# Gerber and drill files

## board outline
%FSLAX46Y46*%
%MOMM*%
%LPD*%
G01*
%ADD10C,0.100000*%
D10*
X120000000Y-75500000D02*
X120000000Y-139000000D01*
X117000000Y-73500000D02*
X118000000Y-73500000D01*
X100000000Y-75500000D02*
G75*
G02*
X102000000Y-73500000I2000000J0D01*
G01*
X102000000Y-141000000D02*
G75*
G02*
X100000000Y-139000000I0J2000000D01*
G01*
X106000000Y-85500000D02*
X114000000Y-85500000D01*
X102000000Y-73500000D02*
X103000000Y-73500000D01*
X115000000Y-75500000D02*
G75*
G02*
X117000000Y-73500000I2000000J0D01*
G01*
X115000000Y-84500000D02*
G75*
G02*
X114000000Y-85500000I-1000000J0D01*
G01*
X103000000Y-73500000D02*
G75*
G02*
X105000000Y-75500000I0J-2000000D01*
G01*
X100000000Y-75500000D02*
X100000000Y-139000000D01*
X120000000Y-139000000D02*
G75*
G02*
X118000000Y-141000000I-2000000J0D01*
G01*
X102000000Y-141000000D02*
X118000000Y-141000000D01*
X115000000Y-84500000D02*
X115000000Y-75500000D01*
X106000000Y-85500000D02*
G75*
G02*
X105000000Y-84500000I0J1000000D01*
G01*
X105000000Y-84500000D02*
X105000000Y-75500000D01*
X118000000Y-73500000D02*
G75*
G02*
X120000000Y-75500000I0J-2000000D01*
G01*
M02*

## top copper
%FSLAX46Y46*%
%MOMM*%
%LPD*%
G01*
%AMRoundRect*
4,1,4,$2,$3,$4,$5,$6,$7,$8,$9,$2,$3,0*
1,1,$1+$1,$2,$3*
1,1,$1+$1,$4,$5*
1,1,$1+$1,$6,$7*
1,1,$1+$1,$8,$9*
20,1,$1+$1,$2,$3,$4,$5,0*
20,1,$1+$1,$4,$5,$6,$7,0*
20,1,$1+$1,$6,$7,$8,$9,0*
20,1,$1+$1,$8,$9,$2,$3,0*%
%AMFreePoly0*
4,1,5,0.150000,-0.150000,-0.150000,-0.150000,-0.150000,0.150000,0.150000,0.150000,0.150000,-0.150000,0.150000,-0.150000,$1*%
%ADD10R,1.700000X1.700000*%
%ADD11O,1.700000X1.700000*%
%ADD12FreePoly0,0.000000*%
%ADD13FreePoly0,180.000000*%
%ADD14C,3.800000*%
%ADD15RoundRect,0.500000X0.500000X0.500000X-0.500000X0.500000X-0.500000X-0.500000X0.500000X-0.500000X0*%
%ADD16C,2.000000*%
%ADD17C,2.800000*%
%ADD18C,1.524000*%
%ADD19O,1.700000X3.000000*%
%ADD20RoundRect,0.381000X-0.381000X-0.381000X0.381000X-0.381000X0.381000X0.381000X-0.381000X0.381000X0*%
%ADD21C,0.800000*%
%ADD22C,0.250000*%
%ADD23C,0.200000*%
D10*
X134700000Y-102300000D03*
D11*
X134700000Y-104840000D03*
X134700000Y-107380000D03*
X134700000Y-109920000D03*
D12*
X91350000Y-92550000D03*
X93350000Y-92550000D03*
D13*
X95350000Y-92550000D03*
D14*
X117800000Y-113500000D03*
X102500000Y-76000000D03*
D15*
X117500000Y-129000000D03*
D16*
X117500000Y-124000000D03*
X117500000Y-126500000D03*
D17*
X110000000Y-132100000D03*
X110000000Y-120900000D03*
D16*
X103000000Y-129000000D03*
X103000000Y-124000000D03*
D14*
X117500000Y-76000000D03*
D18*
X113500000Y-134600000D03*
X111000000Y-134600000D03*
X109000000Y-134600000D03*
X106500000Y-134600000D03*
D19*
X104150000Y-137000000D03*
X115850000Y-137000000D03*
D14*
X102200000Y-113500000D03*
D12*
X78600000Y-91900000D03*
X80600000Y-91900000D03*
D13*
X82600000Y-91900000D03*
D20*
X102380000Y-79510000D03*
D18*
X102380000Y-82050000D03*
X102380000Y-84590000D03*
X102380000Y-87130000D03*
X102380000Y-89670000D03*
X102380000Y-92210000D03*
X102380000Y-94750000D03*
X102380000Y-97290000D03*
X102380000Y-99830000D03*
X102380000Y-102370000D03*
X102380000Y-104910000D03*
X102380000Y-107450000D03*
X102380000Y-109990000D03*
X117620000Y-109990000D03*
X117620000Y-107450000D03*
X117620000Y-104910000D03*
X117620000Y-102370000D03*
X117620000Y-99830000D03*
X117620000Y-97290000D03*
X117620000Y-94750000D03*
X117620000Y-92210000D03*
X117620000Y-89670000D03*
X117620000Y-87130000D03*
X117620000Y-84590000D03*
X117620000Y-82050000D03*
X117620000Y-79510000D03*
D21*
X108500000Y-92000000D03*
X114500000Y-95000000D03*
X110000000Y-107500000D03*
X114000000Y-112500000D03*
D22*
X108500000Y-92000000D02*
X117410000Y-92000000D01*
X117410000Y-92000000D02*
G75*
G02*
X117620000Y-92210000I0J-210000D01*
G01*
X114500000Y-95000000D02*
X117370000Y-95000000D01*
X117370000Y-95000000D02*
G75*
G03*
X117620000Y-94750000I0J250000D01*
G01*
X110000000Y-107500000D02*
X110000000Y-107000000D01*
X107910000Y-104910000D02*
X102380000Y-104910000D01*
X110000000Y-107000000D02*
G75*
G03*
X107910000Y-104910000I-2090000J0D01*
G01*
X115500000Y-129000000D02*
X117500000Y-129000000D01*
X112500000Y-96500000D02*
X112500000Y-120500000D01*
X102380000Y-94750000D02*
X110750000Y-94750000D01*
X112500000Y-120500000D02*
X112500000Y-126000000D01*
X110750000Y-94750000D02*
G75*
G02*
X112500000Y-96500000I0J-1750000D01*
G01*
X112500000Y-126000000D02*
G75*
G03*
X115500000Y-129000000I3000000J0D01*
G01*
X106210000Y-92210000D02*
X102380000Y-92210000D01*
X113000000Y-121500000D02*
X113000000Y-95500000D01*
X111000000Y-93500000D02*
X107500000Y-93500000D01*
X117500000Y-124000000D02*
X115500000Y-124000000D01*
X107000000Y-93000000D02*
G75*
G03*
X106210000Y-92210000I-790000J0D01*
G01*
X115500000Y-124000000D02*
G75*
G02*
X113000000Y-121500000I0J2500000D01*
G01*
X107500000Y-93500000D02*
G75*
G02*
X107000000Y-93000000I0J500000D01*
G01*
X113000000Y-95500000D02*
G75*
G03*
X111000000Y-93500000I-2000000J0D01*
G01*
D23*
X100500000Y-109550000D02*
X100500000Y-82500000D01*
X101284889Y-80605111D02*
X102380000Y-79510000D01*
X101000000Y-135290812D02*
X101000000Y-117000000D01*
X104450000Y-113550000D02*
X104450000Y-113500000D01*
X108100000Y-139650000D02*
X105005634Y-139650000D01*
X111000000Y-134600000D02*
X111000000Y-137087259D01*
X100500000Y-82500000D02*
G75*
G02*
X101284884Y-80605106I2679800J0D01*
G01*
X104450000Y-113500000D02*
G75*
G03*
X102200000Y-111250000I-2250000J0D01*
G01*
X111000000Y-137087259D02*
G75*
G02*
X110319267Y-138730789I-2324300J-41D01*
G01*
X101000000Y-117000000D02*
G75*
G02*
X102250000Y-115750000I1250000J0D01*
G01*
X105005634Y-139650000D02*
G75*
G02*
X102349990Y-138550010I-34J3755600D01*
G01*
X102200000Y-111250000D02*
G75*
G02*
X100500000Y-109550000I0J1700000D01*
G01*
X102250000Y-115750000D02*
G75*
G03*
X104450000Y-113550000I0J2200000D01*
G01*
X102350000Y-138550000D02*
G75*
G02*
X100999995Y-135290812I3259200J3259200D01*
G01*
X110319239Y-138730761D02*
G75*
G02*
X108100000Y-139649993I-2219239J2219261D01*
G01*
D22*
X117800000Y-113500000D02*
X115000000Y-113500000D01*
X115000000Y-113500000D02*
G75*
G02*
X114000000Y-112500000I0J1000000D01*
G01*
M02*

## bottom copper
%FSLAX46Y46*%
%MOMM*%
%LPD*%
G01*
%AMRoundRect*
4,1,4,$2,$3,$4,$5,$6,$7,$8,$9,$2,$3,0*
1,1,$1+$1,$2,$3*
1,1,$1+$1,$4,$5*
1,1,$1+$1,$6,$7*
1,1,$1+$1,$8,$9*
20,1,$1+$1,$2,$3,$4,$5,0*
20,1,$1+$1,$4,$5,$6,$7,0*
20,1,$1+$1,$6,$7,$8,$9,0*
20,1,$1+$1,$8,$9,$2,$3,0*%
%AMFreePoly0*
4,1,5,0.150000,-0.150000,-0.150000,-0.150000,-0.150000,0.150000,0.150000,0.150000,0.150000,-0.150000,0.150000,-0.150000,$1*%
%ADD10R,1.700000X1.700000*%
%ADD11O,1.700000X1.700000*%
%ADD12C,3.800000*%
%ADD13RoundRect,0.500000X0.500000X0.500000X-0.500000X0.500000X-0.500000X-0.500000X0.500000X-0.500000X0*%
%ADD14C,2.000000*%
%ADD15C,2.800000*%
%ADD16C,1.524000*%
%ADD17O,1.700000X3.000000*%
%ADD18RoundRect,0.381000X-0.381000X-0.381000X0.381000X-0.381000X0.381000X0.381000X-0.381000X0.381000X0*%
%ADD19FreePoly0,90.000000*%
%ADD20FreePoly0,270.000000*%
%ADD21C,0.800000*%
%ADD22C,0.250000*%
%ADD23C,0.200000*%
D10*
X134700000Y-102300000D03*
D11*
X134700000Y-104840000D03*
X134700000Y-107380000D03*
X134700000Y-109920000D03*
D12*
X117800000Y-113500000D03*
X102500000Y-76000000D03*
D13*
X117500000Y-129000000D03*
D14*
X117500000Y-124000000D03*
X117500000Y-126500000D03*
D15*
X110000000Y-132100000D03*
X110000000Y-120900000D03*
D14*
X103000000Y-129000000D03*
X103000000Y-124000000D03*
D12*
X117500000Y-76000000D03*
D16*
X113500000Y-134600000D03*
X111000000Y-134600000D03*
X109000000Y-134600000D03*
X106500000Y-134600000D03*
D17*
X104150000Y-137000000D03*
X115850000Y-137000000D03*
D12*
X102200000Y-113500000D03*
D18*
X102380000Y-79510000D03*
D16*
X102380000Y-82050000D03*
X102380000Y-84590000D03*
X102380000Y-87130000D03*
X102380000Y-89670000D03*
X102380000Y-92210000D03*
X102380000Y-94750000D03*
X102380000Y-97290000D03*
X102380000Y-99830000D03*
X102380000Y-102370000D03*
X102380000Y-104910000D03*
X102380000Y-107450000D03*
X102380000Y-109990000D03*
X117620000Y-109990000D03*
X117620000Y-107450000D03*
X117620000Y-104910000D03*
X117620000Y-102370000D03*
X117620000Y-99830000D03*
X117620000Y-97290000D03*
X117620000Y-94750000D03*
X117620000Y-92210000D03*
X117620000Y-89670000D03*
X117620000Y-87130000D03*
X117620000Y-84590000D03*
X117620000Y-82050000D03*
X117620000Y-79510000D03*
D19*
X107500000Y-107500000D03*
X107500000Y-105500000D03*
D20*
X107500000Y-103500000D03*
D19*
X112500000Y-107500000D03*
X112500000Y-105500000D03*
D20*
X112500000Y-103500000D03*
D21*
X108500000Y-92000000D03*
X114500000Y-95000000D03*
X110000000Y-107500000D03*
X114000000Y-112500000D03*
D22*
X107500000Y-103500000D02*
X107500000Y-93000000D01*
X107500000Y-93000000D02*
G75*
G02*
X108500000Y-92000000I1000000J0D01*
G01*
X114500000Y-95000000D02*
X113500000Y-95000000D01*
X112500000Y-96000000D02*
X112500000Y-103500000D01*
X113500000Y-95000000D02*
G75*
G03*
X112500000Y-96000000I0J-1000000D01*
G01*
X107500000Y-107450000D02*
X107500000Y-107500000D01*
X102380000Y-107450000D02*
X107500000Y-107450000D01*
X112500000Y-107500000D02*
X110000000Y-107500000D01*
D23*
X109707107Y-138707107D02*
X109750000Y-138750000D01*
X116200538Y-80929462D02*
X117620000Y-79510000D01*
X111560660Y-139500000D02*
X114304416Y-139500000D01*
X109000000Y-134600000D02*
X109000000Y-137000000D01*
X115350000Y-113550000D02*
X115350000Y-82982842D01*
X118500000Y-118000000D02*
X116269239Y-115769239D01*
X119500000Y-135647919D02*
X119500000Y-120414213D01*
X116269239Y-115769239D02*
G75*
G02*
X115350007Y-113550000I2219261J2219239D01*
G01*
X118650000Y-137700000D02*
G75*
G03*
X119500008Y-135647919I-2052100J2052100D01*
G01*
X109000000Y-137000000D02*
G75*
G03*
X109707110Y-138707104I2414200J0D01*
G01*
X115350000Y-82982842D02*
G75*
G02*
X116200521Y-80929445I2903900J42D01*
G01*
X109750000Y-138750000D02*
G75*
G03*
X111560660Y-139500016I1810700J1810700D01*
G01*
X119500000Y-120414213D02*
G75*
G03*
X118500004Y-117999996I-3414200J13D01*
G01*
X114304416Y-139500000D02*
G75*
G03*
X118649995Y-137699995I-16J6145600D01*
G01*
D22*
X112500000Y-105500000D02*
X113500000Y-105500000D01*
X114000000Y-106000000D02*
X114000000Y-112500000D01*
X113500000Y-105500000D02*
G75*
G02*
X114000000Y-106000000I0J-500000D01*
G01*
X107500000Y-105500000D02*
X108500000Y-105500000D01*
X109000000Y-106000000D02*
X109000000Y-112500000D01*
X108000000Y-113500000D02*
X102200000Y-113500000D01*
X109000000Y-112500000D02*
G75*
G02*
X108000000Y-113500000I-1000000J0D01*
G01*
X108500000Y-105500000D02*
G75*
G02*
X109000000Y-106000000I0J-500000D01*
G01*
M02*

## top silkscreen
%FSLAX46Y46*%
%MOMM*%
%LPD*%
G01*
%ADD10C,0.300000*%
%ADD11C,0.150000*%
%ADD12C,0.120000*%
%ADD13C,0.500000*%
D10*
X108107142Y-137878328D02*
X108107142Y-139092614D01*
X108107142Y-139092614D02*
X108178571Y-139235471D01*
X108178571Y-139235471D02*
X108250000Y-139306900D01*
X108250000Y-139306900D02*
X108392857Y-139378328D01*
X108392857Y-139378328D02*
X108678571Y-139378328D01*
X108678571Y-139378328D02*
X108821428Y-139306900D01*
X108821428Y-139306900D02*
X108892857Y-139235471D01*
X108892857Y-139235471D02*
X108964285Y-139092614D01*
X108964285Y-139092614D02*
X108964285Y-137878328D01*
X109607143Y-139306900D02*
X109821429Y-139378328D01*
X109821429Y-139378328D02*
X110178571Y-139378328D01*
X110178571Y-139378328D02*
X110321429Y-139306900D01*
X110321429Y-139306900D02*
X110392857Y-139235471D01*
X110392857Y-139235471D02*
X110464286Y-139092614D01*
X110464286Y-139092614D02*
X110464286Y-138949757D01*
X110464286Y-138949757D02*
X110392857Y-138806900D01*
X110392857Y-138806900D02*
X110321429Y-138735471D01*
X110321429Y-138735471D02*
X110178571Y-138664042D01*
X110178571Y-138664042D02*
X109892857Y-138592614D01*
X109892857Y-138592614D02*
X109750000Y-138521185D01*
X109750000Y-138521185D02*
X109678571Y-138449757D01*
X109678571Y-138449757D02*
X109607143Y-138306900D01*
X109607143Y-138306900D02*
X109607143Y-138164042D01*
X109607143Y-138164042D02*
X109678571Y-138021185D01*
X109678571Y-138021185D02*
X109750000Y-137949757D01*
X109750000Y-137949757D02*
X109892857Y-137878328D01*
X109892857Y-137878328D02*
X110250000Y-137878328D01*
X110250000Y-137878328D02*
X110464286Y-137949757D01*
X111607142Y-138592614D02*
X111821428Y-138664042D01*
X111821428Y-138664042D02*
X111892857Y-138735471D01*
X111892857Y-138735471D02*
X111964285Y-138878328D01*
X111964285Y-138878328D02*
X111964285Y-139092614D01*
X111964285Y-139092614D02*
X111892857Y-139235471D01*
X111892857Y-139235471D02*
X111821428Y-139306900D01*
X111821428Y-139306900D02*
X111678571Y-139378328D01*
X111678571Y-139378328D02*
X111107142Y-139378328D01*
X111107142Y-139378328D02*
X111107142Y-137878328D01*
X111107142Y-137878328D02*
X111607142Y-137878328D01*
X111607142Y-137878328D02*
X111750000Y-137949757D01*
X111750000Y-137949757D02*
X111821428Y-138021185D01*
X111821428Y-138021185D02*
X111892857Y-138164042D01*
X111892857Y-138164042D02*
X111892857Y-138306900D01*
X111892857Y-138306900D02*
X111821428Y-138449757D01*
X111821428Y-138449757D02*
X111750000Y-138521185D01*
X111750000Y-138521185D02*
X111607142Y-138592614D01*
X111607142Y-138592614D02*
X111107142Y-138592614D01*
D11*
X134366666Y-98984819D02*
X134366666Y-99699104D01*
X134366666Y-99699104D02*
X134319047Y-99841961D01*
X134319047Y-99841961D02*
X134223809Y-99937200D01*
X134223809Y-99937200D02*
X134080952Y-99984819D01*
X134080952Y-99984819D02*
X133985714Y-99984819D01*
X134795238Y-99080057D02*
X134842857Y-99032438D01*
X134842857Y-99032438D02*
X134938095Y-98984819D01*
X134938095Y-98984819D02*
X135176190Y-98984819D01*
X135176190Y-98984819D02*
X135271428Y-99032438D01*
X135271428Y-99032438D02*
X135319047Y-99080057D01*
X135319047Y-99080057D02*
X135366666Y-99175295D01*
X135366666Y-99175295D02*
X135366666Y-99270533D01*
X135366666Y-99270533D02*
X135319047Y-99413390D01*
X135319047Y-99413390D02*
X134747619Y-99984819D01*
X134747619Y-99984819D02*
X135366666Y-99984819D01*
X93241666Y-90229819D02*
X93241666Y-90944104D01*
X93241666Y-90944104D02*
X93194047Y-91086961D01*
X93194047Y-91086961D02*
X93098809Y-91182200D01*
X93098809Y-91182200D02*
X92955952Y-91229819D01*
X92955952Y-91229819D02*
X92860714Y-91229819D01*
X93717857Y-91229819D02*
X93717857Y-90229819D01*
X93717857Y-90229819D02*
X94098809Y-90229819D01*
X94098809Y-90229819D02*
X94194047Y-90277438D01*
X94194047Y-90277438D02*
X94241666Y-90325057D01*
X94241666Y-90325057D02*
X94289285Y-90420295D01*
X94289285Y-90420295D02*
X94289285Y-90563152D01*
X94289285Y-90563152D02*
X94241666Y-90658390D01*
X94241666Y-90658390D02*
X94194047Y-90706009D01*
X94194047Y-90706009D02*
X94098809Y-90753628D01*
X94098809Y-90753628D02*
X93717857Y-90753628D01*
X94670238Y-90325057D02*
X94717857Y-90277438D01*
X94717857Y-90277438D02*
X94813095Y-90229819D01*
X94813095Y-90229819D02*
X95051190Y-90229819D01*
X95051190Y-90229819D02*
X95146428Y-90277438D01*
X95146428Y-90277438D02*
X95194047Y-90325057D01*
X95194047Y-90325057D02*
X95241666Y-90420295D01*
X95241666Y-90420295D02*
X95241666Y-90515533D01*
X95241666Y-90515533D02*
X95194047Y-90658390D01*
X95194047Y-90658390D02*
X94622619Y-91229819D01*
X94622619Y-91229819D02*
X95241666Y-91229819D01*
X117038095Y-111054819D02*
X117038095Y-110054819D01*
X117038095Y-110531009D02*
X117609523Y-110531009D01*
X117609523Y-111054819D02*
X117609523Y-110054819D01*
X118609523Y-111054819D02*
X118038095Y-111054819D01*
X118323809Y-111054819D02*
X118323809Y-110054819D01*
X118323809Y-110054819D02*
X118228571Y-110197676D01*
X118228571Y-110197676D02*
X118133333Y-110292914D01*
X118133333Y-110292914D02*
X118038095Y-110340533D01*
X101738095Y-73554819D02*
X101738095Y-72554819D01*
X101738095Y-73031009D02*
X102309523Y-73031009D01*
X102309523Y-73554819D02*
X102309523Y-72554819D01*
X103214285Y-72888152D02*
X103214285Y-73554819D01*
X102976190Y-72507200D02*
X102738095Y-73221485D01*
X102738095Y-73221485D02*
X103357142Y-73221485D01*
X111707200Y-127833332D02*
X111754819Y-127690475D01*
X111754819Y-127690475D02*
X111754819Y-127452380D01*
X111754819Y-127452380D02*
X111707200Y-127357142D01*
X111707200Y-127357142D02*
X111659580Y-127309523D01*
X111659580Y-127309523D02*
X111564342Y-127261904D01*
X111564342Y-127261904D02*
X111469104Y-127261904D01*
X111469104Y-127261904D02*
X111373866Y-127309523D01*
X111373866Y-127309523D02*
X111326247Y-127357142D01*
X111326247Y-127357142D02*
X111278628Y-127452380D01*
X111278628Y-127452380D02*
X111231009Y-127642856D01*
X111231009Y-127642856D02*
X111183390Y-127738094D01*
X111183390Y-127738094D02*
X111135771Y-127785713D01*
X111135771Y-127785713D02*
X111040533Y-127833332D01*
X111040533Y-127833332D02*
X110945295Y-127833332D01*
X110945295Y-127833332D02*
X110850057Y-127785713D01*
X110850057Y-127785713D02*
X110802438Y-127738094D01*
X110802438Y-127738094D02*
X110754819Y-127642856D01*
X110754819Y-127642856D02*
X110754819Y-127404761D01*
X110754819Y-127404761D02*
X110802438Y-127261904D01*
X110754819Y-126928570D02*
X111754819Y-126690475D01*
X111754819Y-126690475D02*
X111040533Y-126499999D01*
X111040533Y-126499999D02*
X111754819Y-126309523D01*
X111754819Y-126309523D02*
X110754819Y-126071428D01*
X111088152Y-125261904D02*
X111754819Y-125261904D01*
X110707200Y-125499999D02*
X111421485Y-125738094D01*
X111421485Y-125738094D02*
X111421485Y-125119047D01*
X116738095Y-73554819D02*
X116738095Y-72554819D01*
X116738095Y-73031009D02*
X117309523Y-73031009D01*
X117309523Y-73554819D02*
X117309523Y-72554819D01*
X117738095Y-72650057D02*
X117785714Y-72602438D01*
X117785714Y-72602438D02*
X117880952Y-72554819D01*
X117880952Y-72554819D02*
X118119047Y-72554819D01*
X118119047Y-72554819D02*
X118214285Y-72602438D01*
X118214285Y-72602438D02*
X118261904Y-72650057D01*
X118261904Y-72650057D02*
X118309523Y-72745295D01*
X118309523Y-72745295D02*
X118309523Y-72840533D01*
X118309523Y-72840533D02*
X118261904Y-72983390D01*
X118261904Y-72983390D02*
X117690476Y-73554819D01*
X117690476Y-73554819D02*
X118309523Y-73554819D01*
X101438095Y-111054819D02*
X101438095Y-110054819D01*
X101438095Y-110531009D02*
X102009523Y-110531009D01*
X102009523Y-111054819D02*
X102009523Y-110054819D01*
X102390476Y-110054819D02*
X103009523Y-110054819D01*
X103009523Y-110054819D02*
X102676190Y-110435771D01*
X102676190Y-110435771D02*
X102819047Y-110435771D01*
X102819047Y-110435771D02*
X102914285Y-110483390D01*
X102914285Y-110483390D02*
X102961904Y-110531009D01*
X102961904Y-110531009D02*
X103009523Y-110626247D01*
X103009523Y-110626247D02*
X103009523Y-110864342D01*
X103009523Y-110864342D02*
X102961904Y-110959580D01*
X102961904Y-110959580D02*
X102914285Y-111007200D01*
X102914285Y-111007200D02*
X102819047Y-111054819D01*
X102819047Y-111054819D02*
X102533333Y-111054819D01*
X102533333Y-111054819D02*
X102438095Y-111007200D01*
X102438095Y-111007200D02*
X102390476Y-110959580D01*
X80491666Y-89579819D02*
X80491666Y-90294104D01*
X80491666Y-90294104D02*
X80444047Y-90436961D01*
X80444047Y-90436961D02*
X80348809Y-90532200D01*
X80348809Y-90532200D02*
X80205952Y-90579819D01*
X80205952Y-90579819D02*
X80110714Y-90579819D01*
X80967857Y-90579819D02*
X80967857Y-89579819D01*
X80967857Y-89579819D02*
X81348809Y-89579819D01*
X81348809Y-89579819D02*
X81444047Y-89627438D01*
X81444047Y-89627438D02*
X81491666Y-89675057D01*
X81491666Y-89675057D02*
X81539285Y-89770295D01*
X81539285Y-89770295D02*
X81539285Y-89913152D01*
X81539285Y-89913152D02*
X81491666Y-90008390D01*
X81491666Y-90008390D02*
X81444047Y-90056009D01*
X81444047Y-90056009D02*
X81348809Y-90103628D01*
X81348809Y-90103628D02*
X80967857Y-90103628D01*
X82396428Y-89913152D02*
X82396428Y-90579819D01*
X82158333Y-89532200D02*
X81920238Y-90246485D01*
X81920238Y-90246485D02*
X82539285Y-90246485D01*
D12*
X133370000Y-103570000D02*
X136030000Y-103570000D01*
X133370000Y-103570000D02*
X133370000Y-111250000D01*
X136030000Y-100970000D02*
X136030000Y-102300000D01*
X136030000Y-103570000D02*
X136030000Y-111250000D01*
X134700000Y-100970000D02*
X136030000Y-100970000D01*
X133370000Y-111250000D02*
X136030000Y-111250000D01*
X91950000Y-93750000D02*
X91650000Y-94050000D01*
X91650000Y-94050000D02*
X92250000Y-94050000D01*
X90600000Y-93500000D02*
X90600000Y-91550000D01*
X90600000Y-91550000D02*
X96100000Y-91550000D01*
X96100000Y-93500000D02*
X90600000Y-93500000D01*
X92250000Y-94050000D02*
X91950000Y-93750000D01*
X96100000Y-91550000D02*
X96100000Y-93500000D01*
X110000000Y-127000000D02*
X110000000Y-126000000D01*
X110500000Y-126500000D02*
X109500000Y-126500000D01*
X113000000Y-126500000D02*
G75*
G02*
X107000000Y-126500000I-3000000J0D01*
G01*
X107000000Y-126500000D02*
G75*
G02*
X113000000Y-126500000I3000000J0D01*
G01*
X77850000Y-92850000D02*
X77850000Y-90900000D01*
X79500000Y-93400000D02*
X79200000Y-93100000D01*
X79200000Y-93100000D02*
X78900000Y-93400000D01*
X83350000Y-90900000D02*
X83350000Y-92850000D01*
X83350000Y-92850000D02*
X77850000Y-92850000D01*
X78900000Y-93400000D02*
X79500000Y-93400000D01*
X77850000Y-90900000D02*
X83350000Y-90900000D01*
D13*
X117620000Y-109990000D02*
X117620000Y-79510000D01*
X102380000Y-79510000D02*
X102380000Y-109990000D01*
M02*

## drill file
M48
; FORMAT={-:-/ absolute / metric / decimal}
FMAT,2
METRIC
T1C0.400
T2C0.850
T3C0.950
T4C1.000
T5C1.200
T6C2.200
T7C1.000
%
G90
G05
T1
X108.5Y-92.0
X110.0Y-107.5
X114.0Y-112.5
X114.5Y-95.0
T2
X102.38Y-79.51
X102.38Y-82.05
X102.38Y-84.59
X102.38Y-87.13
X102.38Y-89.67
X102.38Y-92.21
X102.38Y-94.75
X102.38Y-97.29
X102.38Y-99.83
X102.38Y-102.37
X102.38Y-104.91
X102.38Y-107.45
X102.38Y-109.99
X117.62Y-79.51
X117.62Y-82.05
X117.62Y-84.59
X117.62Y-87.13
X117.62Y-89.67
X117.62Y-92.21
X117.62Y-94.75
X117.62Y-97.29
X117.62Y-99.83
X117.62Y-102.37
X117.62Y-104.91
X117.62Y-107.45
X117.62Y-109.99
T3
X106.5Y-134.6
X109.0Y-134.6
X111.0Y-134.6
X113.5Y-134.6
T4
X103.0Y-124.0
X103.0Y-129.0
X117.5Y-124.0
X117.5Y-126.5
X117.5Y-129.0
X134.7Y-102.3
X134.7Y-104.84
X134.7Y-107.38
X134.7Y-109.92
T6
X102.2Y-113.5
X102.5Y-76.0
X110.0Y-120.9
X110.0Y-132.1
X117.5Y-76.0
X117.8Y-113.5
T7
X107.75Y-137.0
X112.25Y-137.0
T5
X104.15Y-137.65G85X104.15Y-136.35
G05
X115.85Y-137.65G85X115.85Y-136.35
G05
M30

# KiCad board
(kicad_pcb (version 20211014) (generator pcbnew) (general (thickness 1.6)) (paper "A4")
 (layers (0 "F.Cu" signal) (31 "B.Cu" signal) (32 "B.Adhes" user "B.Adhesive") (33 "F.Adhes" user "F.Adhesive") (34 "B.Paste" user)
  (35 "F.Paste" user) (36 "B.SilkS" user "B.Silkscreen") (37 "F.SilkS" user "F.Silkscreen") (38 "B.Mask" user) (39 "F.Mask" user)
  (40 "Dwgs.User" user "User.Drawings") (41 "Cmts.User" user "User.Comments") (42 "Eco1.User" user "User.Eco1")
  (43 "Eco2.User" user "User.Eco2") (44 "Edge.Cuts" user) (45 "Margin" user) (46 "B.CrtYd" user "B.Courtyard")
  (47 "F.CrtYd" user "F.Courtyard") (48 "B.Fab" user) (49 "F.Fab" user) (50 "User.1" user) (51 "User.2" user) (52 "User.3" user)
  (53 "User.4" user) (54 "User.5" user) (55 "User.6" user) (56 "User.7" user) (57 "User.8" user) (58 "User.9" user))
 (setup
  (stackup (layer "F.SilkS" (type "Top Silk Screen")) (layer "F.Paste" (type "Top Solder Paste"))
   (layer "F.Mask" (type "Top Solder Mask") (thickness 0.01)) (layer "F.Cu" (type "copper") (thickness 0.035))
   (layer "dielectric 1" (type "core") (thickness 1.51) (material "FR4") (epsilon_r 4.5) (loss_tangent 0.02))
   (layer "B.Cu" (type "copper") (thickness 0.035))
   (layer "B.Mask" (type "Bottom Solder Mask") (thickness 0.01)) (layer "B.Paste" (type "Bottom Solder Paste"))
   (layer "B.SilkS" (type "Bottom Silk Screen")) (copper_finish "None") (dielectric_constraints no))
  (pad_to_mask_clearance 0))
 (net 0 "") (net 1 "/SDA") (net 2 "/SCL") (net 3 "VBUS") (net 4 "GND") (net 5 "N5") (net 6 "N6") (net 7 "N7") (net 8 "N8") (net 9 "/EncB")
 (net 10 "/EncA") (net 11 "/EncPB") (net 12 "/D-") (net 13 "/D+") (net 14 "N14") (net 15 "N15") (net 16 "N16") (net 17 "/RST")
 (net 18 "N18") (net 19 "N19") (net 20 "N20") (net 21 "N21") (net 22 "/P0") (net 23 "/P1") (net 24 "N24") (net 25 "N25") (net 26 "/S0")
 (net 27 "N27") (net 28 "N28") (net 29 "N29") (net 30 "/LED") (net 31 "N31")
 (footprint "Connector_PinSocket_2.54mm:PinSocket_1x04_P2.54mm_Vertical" (layer "F.Cu") (at 134.7 102.3)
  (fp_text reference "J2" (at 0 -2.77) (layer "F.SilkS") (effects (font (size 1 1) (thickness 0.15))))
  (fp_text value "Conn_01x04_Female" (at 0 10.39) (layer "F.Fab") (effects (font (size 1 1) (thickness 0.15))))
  (fp_line (start -1.33 1.27) (end 1.33 1.27) (layer "F.SilkS") (width 0.12))
  (fp_line (start -1.33 1.27) (end -1.33 8.95) (layer "F.SilkS") (width 0.12))
  (fp_line (start 1.33 -1.33) (end 1.33 0) (layer "F.SilkS") (width 0.12))
  (fp_line (start 1.33 1.27) (end 1.33 8.95) (layer "F.SilkS") (width 0.12))
  (fp_line (start 0 -1.33) (end 1.33 -1.33) (layer "F.SilkS") (width 0.12))
  (fp_line (start -1.33 8.95) (end 1.33 8.95) (layer "F.SilkS") (width 0.12))
  (pad "1" thru_hole rect (at 0 0) (size 1.7 1.7) (drill 1) (layers *.Cu *.Mask) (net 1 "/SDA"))
  (pad "2" thru_hole oval (at 0 2.54) (size 1.7 1.7) (drill 1) (layers *.Cu *.Mask) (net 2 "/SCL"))
  (pad "3" thru_hole oval (at 0 5.08) (size 1.7 1.7) (drill 1) (layers *.Cu *.Mask) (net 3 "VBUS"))
  (pad "4" thru_hole oval (at 0 7.62) (size 1.7 1.7) (drill 1) (layers *.Cu *.Mask) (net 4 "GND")))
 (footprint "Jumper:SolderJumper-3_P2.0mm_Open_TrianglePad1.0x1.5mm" (layer "F.Cu") (at 93.35 92.55)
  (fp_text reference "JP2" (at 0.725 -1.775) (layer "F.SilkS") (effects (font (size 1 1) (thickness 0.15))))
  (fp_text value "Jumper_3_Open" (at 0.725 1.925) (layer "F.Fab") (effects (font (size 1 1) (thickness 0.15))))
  (fp_line (start -1.4 1.2) (end -1.7 1.5) (layer "F.SilkS") (width 0.12))
  (fp_line (start -1.7 1.5) (end -1.1 1.5) (layer "F.SilkS") (width 0.12))
  (fp_line (start -2.75 0.95) (end -2.75 -1) (layer "F.SilkS") (width 0.12))
  (fp_line (start -2.75 -1) (end 2.75 -1) (layer "F.SilkS") (width 0.12))
  (fp_line (start 2.75 0.95) (end -2.75 0.95) (layer "F.SilkS") (width 0.12))
  (fp_line (start -1.1 1.5) (end -1.4 1.2) (layer "F.SilkS") (width 0.12))
  (fp_line (start 2.75 -1) (end 2.75 0.95) (layer "F.SilkS") (width 0.12))
  (pad "" smd rect (at 1.2 0) (size 1.5 1.5) (layers "F.Mask"))
  (pad "" smd rect (at -1.2 0) (size 1.5 1.5) (layers "F.Mask"))
  (pad "1" smd custom (at -2 0) (size 0.3 0.3) (layers "F.Cu" "F.Mask") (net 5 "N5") (zone_connect 2)
   (options (clearance outline) (anchor rect)) (primitives))
  (pad "2" smd custom (at 0 0) (size 0.3 0.3) (layers "F.Cu") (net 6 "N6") (zone_connect 2) (options (clearance outline) (anchor rect))
   (primitives))
  (pad "3" smd custom (at 2 0 180) (size 0.3 0.3) (layers "F.Cu" "F.Mask") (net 3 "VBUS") (zone_connect 2)
   (options (clearance outline) (anchor rect)) (primitives)))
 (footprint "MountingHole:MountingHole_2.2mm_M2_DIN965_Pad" (layer "F.Cu") (at 117.8 113.5)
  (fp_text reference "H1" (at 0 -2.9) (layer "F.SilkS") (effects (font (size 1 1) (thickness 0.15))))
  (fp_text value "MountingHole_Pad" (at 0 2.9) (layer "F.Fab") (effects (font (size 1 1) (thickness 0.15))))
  (pad "1" thru_hole circle (at 0 0) (size 3.8 3.8) (drill 2.2) (layers *.Cu *.Mask) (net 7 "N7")))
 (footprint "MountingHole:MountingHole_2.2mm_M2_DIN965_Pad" (layer "F.Cu") (at 102.5 76)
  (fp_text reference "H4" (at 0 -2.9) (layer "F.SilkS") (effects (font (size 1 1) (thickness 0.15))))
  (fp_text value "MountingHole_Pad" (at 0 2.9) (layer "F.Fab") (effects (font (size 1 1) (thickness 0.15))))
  (pad "1" thru_hole circle (at 0 0) (size 3.8 3.8) (drill 2.2) (layers *.Cu *.Mask) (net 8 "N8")))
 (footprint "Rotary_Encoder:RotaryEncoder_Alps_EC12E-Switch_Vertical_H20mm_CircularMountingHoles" (layer "F.Cu") (at 117.5 129 180)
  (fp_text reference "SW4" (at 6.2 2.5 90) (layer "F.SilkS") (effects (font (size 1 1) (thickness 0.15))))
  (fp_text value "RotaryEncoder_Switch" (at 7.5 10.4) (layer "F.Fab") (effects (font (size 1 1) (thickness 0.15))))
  (fp_line (start 7.5 2) (end 7.5 3) (layer "F.SilkS") (width 0.12))
  (fp_line (start 7 2.5) (end 8 2.5) (layer "F.SilkS") (width 0.12))
  (fp_circle (center 7.5 2.5) (end 10.5 2.5) (layer "F.SilkS") (width 0.12) (fill none))
  (pad "A" thru_hole roundrect (at 0 0 180) (size 2 2) (drill 1) (layers *.Cu *.Mask) (roundrect_rratio 0.25) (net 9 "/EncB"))
  (pad "B" thru_hole circle (at 0 5 180) (size 2 2) (drill 1) (layers *.Cu *.Mask) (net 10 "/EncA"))
  (pad "C" thru_hole circle (at 0 2.5 180) (size 2 2) (drill 1) (layers *.Cu *.Mask) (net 4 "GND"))
  (pad "MP" thru_hole circle (at 7.5 -3.1 180) (size 2.8 2.8) (drill 2.2) (layers *.Cu *.Mask))
  (pad "MP" thru_hole circle (at 7.5 8.1 180) (size 2.8 2.8) (drill 2.2) (layers *.Cu *.Mask))
  (pad "S1" thru_hole circle (at 14.5 0 180) (size 2 2) (drill 1) (layers *.Cu *.Mask) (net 4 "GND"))
  (pad "S2" thru_hole circle (at 14.5 5 180) (size 2 2) (drill 1) (layers *.Cu *.Mask) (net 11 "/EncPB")))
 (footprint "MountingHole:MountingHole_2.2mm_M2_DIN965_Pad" (layer "F.Cu") (at 117.5 76)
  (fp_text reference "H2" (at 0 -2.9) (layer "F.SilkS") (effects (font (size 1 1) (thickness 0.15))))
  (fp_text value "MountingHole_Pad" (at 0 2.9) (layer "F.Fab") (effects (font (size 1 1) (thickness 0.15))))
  (pad "1" thru_hole circle (at 0 0) (size 3.8 3.8) (drill 2.2) (layers *.Cu *.Mask) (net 6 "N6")))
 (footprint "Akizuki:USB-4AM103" (layer "F.Cu") (at 110 136 180)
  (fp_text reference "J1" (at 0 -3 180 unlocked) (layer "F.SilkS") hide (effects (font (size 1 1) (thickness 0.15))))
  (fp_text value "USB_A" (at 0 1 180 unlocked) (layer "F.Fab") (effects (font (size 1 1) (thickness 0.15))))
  (pad "" np_thru_hole circle (at 2.25 -1 180) (size 1 1) (drill 1) (layers *.Mask))
  (pad "" np_thru_hole circle (at -2.25 -1 180) (size 1 1) (drill 1) (layers *.Mask))
  (pad "1" thru_hole circle (at -3.5 1.4 180) (size 1.524 1.524) (drill 0.95) (layers *.Cu *.Mask) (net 3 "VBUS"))
  (pad "2" thru_hole circle (at -1 1.4 180) (size 1.524 1.524) (drill 0.95) (layers *.Cu *.Mask) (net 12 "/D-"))
  (pad "3" thru_hole circle (at 1 1.4 180) (size 1.524 1.524) (drill 0.95) (layers *.Cu *.Mask) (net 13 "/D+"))
  (pad "4" thru_hole circle (at 3.5 1.4 180) (size 1.524 1.524) (drill 0.95) (layers *.Cu *.Mask) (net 4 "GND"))
  (pad "5" thru_hole oval (at 5.85 -1 180) (size 1.7 3) (drill oval 1.2 2.5) (layers *.Cu *.Mask) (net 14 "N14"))
  (pad "5" thru_hole oval (at -5.85 -1 180) (size 1.7 3) (drill oval 1.2 2.5) (layers *.Cu *.Mask) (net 14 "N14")))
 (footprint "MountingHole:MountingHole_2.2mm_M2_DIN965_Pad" (layer "F.Cu") (at 102.2 113.5)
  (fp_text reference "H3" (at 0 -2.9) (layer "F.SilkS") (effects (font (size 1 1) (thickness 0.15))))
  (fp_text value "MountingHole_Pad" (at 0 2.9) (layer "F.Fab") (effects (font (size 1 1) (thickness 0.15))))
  (pad "1" thru_hole circle (at 0 0) (size 3.8 3.8) (drill 2.2) (layers *.Cu *.Mask) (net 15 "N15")))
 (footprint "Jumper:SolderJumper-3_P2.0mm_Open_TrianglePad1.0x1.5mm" (layer "F.Cu") (at 80.6 91.9)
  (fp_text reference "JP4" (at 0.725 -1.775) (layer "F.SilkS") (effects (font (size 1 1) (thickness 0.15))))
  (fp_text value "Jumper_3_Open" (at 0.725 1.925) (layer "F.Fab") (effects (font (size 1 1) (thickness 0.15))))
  (fp_line (start -2.75 0.95) (end -2.75 -1) (layer "F.SilkS") (width 0.12))
  (fp_line (start -1.1 1.5) (end -1.4 1.2) (layer "F.SilkS") (width 0.12))
  (fp_line (start -1.4 1.2) (end -1.7 1.5) (layer "F.SilkS") (width 0.12))
  (fp_line (start 2.75 -1) (end 2.75 0.95) (layer "F.SilkS") (width 0.12))
  (fp_line (start 2.75 0.95) (end -2.75 0.95) (layer "F.SilkS") (width 0.12))
  (fp_line (start -1.7 1.5) (end -1.1 1.5) (layer "F.SilkS") (width 0.12))
  (fp_line (start -2.75 -1) (end 2.75 -1) (layer "F.SilkS") (width 0.12))
  (pad "" smd rect (at -1.2 0) (size 1.5 1.5) (layers "F.Mask"))
  (pad "" smd rect (at 1.2 0) (size 1.5 1.5) (layers "F.Mask"))
  (pad "1" smd custom (at -2 0) (size 0.3 0.3) (layers "F.Cu" "F.Mask") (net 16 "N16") (zone_connect 2)
   (options (clearance outline) (anchor rect)) (primitives))
  (pad "2" smd custom (at 0 0) (size 0.3 0.3) (layers "F.Cu") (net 8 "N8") (zone_connect 2) (options (clearance outline) (anchor rect))
   (primitives))
  (pad "3" smd custom (at 2 0 180) (size 0.3 0.3) (layers "F.Cu" "F.Mask") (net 4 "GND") (zone_connect 2)
   (options (clearance outline) (anchor rect)) (primitives)))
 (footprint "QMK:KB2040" (layer "F.Cu") (at 110 94.75)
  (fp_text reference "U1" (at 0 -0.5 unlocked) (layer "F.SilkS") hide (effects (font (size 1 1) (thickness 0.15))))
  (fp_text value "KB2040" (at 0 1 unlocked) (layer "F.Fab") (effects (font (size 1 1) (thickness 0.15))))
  (fp_line (start 7.62 15.24) (end 7.62 -15.24) (layer "F.SilkS") (width 0.5))
  (fp_line (start -7.62 -15.24) (end -7.62 15.24) (layer "F.SilkS") (width 0.5))
  (pad "0" thru_hole roundrect (at -7.62 -15.24) (size 1.524 1.524) (drill 0.85) (layers *.Cu *.Mask) (roundrect_rratio 0.25) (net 12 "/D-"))
  (pad "1" thru_hole circle (at -7.62 -12.7) (size 1.524 1.524) (drill 0.85) (layers *.Cu *.Mask) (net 3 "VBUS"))
  (pad "2" thru_hole circle (at -7.62 -10.16) (size 1.524 1.524) (drill 0.85) (layers *.Cu *.Mask) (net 4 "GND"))
  (pad "3" thru_hole circle (at -7.62 -7.62) (size 1.524 1.524) (drill 0.85) (layers *.Cu *.Mask) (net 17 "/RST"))
  (pad "4" thru_hole circle (at -7.62 -5.08) (size 1.524 1.524) (drill 0.85) (layers *.Cu *.Mask) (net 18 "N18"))
  (pad "5" thru_hole circle (at -7.62 -2.54) (size 1.524 1.524) (drill 0.85) (layers *.Cu *.Mask) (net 10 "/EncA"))
  (pad "6" thru_hole circle (at -7.62 0) (size 1.524 1.524) (drill 0.85) (layers *.Cu *.Mask) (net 9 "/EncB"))
  (pad "7" thru_hole circle (at -7.62 2.54) (size 1.524 1.524) (drill 0.85) (layers *.Cu *.Mask) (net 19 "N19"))
  (pad "8" thru_hole circle (at -7.62 5.08) (size 1.524 1.524) (drill 0.85) (layers *.Cu *.Mask) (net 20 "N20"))
  (pad "9" thru_hole circle (at -7.62 7.62) (size 1.524 1.524) (drill 0.85) (layers *.Cu *.Mask) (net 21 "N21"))
  (pad "10" thru_hole circle (at -7.62 10.16) (size 1.524 1.524) (drill 0.85) (layers *.Cu *.Mask) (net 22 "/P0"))
  (pad "11" thru_hole circle (at -7.62 12.7) (size 1.524 1.524) (drill 0.85) (layers *.Cu *.Mask) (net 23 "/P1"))
  (pad "12" thru_hole circle (at -7.62 15.24) (size 1.524 1.524) (drill 0.85) (layers *.Cu *.Mask) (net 11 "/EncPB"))
  (pad "13" thru_hole circle (at 7.62 15.24) (size 1.524 1.524) (drill 0.85) (layers *.Cu *.Mask) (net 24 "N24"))
  (pad "14" thru_hole circle (at 7.62 12.7) (size 1.524 1.524) (drill 0.85) (layers *.Cu *.Mask) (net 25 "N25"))
  (pad "15" thru_hole circle (at 7.62 10.16) (size 1.524 1.524) (drill 0.85) (layers *.Cu *.Mask) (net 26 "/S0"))
  (pad "16" thru_hole circle (at 7.62 7.62) (size 1.524 1.524) (drill 0.85) (layers *.Cu *.Mask) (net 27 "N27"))
  (pad "17" thru_hole circle (at 7.62 5.08) (size 1.524 1.524) (drill 0.85) (layers *.Cu *.Mask) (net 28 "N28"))
  (pad "18" thru_hole circle (at 7.62 2.54) (size 1.524 1.524) (drill 0.85) (layers *.Cu *.Mask) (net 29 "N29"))
  (pad "19" thru_hole circle (at 7.62 0) (size 1.524 1.524) (drill 0.85) (layers *.Cu *.Mask) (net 2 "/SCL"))
  (pad "20" thru_hole circle (at 7.62 -2.54) (size 1.524 1.524) (drill 0.85) (layers *.Cu *.Mask) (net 1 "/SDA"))
  (pad "21" thru_hole circle (at 7.62 -5.08) (size 1.524 1.524) (drill 0.85) (layers *.Cu *.Mask) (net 4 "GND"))
  (pad "22" thru_hole circle (at 7.62 -7.62) (size 1.524 1.524) (drill 0.85) (layers *.Cu *.Mask) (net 4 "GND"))
  (pad "23" thru_hole circle (at 7.62 -10.16) (size 1.524 1.524) (drill 0.85) (layers *.Cu *.Mask) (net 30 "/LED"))
  (pad "24" thru_hole circle (at 7.62 -12.7) (size 1.524 1.524) (drill 0.85) (layers *.Cu *.Mask) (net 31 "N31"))
  (pad "25" thru_hole circle (at 7.62 -15.24) (size 1.524 1.524) (drill 0.85) (layers *.Cu *.Mask) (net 13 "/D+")))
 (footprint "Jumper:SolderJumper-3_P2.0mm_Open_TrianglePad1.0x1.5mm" (layer "B.Cu") (at 107.5 105.5 90)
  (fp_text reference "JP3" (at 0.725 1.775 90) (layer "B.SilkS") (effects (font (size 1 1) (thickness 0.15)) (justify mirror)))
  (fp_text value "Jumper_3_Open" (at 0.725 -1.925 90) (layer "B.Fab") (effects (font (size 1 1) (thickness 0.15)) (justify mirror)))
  (pad "" smd rect (at 1.2 0 90) (size 1.5 1.5) (layers "B.Mask"))
  (pad "" smd rect (at -1.2 0 90) (size 1.5 1.5) (layers "B.Mask"))
  (pad "1" smd custom (at -2 0 90) (size 0.3 0.3) (layers "B.Cu" "B.Mask") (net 23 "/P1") (zone_connect 2)
   (options (clearance outline) (anchor rect)) (primitives))
  (pad "2" smd custom (at 0 0 90) (size 0.3 0.3) (layers "B.Cu") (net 15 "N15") (zone_connect 2) (options (clearance outline) (anchor rect))
   (primitives))
  (pad "3" smd custom (at 2 0 270) (size 0.3 0.3) (layers "B.Cu" "B.Mask") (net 1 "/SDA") (zone_connect 2)
   (options (clearance outline) (anchor rect)) (primitives)))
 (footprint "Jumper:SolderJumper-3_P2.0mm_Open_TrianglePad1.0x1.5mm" (layer "B.Cu") (at 112.5 105.5 90)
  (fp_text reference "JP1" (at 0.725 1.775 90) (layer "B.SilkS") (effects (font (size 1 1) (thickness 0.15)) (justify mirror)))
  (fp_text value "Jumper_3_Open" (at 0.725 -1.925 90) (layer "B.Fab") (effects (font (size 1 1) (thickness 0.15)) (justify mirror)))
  (pad "" smd rect (at -1.2 0 90) (size 1.5 1.5) (layers "B.Mask"))
  (pad "" smd rect (at 1.2 0 90) (size 1.5 1.5) (layers "B.Mask"))
  (pad "1" smd custom (at -2 0 90) (size 0.3 0.3) (layers "B.Cu" "B.Mask") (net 22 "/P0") (zone_connect 2)
   (options (clearance outline) (anchor rect)) (primitives))
  (pad "2" smd custom (at 0 0 90) (size 0.3 0.3) (layers "B.Cu") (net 7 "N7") (zone_connect 2) (options (clearance outline) (anchor rect))
   (primitives))
  (pad "3" smd custom (at 2 0 270) (size 0.3 0.3) (layers "B.Cu" "B.Mask") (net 2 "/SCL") (zone_connect 2)
   (options (clearance outline) (anchor rect)) (primitives)))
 (gr_line (start 120 75.5) (end 120 139) (layer "Edge.Cuts") (width 0.1))
 (gr_line (start 117 73.5) (end 118 73.5) (layer "Edge.Cuts") (width 0.1))
 (gr_arc (start 100 75.5) (mid 100.585786 74.085786) (end 102 73.5) (layer "Edge.Cuts") (width 0.1))
 (gr_arc (start 102 141) (mid 100.585786 140.414214) (end 100 139) (layer "Edge.Cuts") (width 0.1))
 (gr_line (start 106 85.5) (end 114 85.5) (layer "Edge.Cuts") (width 0.1))
 (gr_line (start 102 73.5) (end 103 73.5) (layer "Edge.Cuts") (width 0.1))
 (gr_arc (start 115 75.5) (mid 115.585786 74.085786) (end 117 73.5) (layer "Edge.Cuts") (width 0.1))
 (gr_arc (start 115 84.5) (mid 114.707107 85.207107) (end 114 85.5) (layer "Edge.Cuts") (width 0.1))
 (gr_arc (start 103 73.5) (mid 104.414214 74.085786) (end 105 75.5) (layer "Edge.Cuts") (width 0.1))
 (gr_line (start 100 75.5) (end 100 139) (layer "Edge.Cuts") (width 0.1))
 (gr_arc (start 120 139) (mid 119.414214 140.414214) (end 118 141) (layer "Edge.Cuts") (width 0.1))
 (gr_line (start 102 141) (end 118 141) (layer "Edge.Cuts") (width 0.1))
 (gr_line (start 115 84.5) (end 115 75.5) (layer "Edge.Cuts") (width 0.1))
 (gr_arc (start 106 85.5) (mid 105.292893 85.207107) (end 105 84.5) (layer "Edge.Cuts") (width 0.1))
 (gr_line (start 105 84.5) (end 105 75.5) (layer "Edge.Cuts") (width 0.1))
 (gr_arc (start 118 73.5) (mid 119.414214 74.085786) (end 120 75.5) (layer "Edge.Cuts") (width 0.1))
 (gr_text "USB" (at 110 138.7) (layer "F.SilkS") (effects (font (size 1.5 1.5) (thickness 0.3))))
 (segment (start 108.5 92) (end 117.41 92) (width 0.25) (layer "F.Cu") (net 1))
 (via (at 108.5 92) (size 0.8) (drill 0.4) (layers "F.Cu" "B.Cu") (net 1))
 (arc (start 117.41 92) (mid 117.558492 92.061508) (end 117.62 92.21) (width 0.25) (layer "F.Cu") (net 1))
 (segment (start 107.5 103.5) (end 107.5 93) (width 0.25) (layer "B.Cu") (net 1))
 (arc (start 107.5 93) (mid 107.792893 92.292893) (end 108.5 92) (width 0.25) (layer "B.Cu") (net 1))
 (segment (start 114.5 95) (end 117.37 95) (width 0.25) (layer "F.Cu") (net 2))
 (via (at 114.5 95) (size 0.8) (drill 0.4) (layers "F.Cu" "B.Cu") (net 2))
 (arc (start 117.37 95) (mid 117.546777 94.926777) (end 117.62 94.75) (width 0.25) (layer "F.Cu") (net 2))
 (segment (start 114.5 95) (end 113.5 95) (width 0.25) (layer "B.Cu") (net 2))
 (segment (start 112.5 96) (end 112.5 103.5) (width 0.25) (layer "B.Cu") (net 2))
 (arc (start 113.5 95) (mid 112.792893 95.292893) (end 112.5 96) (width 0.25) (layer "B.Cu") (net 2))
 (segment (start 107.5 107.45) (end 107.5 107.5) (width 0.25) (layer "B.Cu") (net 23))
 (segment (start 102.38 107.45) (end 107.5 107.45) (width 0.25) (layer "B.Cu") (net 23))
 (segment (start 110 107.5) (end 110 107) (width 0.25) (layer "F.Cu") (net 22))
 (segment (start 107.91 104.91) (end 102.38 104.91) (width 0.25) (layer "F.Cu") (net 22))
 (via (at 110 107.5) (size 0.8) (drill 0.4) (layers "F.Cu" "B.Cu") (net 22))
 (arc (start 110 107) (mid 109.387853 105.522147) (end 107.91 104.91) (width 0.25) (layer "F.Cu") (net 22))
 (segment (start 112.5 107.5) (end 110 107.5) (width 0.25) (layer "B.Cu") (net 22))
 (segment (start 115.5 129) (end 117.5 129) (width 0.25) (layer "F.Cu") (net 9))
 (segment (start 112.5 96.5) (end 112.5 120.5) (width 0.25) (layer "F.Cu") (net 9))
 (segment (start 102.38 94.75) (end 110.75 94.75) (width 0.25) (layer "F.Cu") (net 9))
 (segment (start 112.5 120.5) (end 112.5 126) (width 0.25) (layer "F.Cu") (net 9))
 (arc (start 110.75 94.75) (mid 111.987437 95.262563) (end 112.5 96.5) (width 0.25) (layer "F.Cu") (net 9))
 (arc (start 112.5 126) (mid 113.37868 128.12132) (end 115.5 129) (width 0.25) (layer "F.Cu") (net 9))
 (segment (start 106.21 92.21) (end 102.38 92.21) (width 0.25) (layer "F.Cu") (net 10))
 (segment (start 113 121.5) (end 113 95.5) (width 0.25) (layer "F.Cu") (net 10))
 (segment (start 111 93.5) (end 107.5 93.5) (width 0.25) (layer "F.Cu") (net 10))
 (segment (start 117.5 124) (end 115.5 124) (width 0.25) (layer "F.Cu") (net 10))
 (arc (start 107 93) (mid 106.768614 92.441386) (end 106.21 92.21) (width 0.25) (layer "F.Cu") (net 10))
 (arc (start 115.5 124) (mid 113.732233 123.267767) (end 113 121.5) (width 0.25) (layer "F.Cu") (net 10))
 (arc (start 107.5 93.5) (mid 107.146447 93.353553) (end 107 93) (width 0.25) (layer "F.Cu") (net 10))
 (arc (start 113 95.5) (mid 112.414214 94.085786) (end 111 93.5) (width 0.25) (layer "F.Cu") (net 10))
 (segment (start 100.5 109.55) (end 100.5 82.5) (width 0.2) (layer "F.Cu") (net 12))
 (segment (start 101.284889 80.605111) (end 102.38 79.51) (width 0.2) (layer "F.Cu") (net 12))
 (segment (start 101 135.290812) (end 101 117) (width 0.2) (layer "F.Cu") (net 12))
 (segment (start 104.45 113.55) (end 104.45 113.5) (width 0.2) (layer "F.Cu") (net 12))
 (segment (start 108.1 139.65) (end 105.005634 139.65) (width 0.2) (layer "F.Cu") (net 12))
 (segment (start 111 134.6) (end 111 137.087259) (width 0.2) (layer "F.Cu") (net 12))
 (arc (start 100.5 82.5) (mid 100.703986 81.474493) (end 101.284889 80.605111) (width 0.2) (layer "F.Cu") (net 12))
 (arc (start 104.45 113.5) (mid 103.79099 111.90901) (end 102.2 111.25) (width 0.2) (layer "F.Cu") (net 12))
 (arc (start 111 137.087259) (mid 110.823076 137.976716) (end 110.319239 138.730761) (width 0.2) (layer "F.Cu") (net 12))
 (arc (start 101 117) (mid 101.366117 116.116117) (end 102.25 115.75) (width 0.2) (layer "F.Cu") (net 12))
 (arc (start 105.005634 139.65) (mid 103.568415 139.364119) (end 102.35 138.55) (width 0.2) (layer "F.Cu") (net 12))
 (arc (start 102.2 111.25) (mid 100.997918 110.752082) (end 100.5 109.55) (width 0.2) (layer "F.Cu") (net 12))
 (arc (start 102.25 115.75) (mid 103.805635 115.105635) (end 104.45 113.55) (width 0.2) (layer "F.Cu") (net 12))
 (arc (start 102.35 138.55) (mid 101.350854 137.054671) (end 101 135.290812) (width 0.2) (layer "F.Cu") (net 12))
 (arc (start 110.319239 138.730761) (mid 109.301044 139.411098) (end 108.1 139.65) (width 0.2) (layer "F.Cu") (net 12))
 (segment (start 109.707107 138.707107) (end 109.75 138.75) (width 0.2) (layer "B.Cu") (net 13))
 (segment (start 116.200538 80.929462) (end 117.62 79.51) (width 0.2) (layer "B.Cu") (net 13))
 (segment (start 111.56066 139.5) (end 114.304416 139.5) (width 0.2) (layer "B.Cu") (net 13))
 (segment (start 109 134.6) (end 109 137) (width 0.2) (layer "B.Cu") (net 13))
 (segment (start 115.35 113.55) (end 115.35 82.982842) (width 0.2) (layer "B.Cu") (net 13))
 (segment (start 118.5 118) (end 116.269239 115.769239) (width 0.2) (layer "B.Cu") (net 13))
 (segment (start 119.5 135.647919) (end 119.5 120.414213) (width 0.2) (layer "B.Cu") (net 13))
 (arc (start 116.269239 115.769239) (mid 115.588902 114.751044) (end 115.35 113.55) (width 0.2) (layer "B.Cu") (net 13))
 (arc (start 118.65 137.7) (mid 119.279092 136.758497) (end 119.5 135.647919) (width 0.2) (layer "B.Cu") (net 13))
 (arc (start 109 137) (mid 109.183771 137.92388) (end 109.707107 138.707107) (width 0.2) (layer "B.Cu") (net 13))
 (arc (start 115.35 82.982842) (mid 115.571048 81.871561) (end 116.200538 80.929462) (width 0.2) (layer "B.Cu") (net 13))
 (arc (start 109.75 138.75) (mid 110.580738 139.305081) (end 111.56066 139.5) (width 0.2) (layer "B.Cu") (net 13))
 (arc (start 119.5 120.414213) (mid 119.240108 119.10765) (end 118.5 118) (width 0.2) (layer "B.Cu") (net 13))
 (arc (start 114.304416 139.5) (mid 116.656229 139.032195) (end 118.65 137.7) (width 0.2) (layer "B.Cu") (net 13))
 (segment (start 117.8 113.5) (end 115 113.5) (width 0.25) (layer "F.Cu") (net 7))
 (via (at 114 112.5) (size 0.8) (drill 0.4) (layers "F.Cu" "B.Cu") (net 7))
 (arc (start 115 113.5) (mid 114.292893 113.207107) (end 114 112.5) (width 0.25) (layer "F.Cu") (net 7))
 (segment (start 112.5 105.5) (end 113.5 105.5) (width 0.25) (layer "B.Cu") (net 7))
 (segment (start 114 106) (end 114 112.5) (width 0.25) (layer "B.Cu") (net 7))
 (arc (start 113.5 105.5) (mid 113.853553 105.646447) (end 114 106) (width 0.25) (layer "B.Cu") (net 7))
 (segment (start 107.5 105.5) (end 108.5 105.5) (width 0.25) (layer "B.Cu") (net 15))
 (segment (start 109 106) (end 109 112.5) (width 0.25) (layer "B.Cu") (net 15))
 (segment (start 108 113.5) (end 102.2 113.5) (width 0.25) (layer "B.Cu") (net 15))
 (arc (start 109 112.5) (mid 108.707107 113.207107) (end 108 113.5) (width 0.25) (layer "B.Cu") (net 15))
 (arc (start 108.5 105.5) (mid 108.853553 105.646447) (end 109 106) (width 0.25) (layer "B.Cu") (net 15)))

